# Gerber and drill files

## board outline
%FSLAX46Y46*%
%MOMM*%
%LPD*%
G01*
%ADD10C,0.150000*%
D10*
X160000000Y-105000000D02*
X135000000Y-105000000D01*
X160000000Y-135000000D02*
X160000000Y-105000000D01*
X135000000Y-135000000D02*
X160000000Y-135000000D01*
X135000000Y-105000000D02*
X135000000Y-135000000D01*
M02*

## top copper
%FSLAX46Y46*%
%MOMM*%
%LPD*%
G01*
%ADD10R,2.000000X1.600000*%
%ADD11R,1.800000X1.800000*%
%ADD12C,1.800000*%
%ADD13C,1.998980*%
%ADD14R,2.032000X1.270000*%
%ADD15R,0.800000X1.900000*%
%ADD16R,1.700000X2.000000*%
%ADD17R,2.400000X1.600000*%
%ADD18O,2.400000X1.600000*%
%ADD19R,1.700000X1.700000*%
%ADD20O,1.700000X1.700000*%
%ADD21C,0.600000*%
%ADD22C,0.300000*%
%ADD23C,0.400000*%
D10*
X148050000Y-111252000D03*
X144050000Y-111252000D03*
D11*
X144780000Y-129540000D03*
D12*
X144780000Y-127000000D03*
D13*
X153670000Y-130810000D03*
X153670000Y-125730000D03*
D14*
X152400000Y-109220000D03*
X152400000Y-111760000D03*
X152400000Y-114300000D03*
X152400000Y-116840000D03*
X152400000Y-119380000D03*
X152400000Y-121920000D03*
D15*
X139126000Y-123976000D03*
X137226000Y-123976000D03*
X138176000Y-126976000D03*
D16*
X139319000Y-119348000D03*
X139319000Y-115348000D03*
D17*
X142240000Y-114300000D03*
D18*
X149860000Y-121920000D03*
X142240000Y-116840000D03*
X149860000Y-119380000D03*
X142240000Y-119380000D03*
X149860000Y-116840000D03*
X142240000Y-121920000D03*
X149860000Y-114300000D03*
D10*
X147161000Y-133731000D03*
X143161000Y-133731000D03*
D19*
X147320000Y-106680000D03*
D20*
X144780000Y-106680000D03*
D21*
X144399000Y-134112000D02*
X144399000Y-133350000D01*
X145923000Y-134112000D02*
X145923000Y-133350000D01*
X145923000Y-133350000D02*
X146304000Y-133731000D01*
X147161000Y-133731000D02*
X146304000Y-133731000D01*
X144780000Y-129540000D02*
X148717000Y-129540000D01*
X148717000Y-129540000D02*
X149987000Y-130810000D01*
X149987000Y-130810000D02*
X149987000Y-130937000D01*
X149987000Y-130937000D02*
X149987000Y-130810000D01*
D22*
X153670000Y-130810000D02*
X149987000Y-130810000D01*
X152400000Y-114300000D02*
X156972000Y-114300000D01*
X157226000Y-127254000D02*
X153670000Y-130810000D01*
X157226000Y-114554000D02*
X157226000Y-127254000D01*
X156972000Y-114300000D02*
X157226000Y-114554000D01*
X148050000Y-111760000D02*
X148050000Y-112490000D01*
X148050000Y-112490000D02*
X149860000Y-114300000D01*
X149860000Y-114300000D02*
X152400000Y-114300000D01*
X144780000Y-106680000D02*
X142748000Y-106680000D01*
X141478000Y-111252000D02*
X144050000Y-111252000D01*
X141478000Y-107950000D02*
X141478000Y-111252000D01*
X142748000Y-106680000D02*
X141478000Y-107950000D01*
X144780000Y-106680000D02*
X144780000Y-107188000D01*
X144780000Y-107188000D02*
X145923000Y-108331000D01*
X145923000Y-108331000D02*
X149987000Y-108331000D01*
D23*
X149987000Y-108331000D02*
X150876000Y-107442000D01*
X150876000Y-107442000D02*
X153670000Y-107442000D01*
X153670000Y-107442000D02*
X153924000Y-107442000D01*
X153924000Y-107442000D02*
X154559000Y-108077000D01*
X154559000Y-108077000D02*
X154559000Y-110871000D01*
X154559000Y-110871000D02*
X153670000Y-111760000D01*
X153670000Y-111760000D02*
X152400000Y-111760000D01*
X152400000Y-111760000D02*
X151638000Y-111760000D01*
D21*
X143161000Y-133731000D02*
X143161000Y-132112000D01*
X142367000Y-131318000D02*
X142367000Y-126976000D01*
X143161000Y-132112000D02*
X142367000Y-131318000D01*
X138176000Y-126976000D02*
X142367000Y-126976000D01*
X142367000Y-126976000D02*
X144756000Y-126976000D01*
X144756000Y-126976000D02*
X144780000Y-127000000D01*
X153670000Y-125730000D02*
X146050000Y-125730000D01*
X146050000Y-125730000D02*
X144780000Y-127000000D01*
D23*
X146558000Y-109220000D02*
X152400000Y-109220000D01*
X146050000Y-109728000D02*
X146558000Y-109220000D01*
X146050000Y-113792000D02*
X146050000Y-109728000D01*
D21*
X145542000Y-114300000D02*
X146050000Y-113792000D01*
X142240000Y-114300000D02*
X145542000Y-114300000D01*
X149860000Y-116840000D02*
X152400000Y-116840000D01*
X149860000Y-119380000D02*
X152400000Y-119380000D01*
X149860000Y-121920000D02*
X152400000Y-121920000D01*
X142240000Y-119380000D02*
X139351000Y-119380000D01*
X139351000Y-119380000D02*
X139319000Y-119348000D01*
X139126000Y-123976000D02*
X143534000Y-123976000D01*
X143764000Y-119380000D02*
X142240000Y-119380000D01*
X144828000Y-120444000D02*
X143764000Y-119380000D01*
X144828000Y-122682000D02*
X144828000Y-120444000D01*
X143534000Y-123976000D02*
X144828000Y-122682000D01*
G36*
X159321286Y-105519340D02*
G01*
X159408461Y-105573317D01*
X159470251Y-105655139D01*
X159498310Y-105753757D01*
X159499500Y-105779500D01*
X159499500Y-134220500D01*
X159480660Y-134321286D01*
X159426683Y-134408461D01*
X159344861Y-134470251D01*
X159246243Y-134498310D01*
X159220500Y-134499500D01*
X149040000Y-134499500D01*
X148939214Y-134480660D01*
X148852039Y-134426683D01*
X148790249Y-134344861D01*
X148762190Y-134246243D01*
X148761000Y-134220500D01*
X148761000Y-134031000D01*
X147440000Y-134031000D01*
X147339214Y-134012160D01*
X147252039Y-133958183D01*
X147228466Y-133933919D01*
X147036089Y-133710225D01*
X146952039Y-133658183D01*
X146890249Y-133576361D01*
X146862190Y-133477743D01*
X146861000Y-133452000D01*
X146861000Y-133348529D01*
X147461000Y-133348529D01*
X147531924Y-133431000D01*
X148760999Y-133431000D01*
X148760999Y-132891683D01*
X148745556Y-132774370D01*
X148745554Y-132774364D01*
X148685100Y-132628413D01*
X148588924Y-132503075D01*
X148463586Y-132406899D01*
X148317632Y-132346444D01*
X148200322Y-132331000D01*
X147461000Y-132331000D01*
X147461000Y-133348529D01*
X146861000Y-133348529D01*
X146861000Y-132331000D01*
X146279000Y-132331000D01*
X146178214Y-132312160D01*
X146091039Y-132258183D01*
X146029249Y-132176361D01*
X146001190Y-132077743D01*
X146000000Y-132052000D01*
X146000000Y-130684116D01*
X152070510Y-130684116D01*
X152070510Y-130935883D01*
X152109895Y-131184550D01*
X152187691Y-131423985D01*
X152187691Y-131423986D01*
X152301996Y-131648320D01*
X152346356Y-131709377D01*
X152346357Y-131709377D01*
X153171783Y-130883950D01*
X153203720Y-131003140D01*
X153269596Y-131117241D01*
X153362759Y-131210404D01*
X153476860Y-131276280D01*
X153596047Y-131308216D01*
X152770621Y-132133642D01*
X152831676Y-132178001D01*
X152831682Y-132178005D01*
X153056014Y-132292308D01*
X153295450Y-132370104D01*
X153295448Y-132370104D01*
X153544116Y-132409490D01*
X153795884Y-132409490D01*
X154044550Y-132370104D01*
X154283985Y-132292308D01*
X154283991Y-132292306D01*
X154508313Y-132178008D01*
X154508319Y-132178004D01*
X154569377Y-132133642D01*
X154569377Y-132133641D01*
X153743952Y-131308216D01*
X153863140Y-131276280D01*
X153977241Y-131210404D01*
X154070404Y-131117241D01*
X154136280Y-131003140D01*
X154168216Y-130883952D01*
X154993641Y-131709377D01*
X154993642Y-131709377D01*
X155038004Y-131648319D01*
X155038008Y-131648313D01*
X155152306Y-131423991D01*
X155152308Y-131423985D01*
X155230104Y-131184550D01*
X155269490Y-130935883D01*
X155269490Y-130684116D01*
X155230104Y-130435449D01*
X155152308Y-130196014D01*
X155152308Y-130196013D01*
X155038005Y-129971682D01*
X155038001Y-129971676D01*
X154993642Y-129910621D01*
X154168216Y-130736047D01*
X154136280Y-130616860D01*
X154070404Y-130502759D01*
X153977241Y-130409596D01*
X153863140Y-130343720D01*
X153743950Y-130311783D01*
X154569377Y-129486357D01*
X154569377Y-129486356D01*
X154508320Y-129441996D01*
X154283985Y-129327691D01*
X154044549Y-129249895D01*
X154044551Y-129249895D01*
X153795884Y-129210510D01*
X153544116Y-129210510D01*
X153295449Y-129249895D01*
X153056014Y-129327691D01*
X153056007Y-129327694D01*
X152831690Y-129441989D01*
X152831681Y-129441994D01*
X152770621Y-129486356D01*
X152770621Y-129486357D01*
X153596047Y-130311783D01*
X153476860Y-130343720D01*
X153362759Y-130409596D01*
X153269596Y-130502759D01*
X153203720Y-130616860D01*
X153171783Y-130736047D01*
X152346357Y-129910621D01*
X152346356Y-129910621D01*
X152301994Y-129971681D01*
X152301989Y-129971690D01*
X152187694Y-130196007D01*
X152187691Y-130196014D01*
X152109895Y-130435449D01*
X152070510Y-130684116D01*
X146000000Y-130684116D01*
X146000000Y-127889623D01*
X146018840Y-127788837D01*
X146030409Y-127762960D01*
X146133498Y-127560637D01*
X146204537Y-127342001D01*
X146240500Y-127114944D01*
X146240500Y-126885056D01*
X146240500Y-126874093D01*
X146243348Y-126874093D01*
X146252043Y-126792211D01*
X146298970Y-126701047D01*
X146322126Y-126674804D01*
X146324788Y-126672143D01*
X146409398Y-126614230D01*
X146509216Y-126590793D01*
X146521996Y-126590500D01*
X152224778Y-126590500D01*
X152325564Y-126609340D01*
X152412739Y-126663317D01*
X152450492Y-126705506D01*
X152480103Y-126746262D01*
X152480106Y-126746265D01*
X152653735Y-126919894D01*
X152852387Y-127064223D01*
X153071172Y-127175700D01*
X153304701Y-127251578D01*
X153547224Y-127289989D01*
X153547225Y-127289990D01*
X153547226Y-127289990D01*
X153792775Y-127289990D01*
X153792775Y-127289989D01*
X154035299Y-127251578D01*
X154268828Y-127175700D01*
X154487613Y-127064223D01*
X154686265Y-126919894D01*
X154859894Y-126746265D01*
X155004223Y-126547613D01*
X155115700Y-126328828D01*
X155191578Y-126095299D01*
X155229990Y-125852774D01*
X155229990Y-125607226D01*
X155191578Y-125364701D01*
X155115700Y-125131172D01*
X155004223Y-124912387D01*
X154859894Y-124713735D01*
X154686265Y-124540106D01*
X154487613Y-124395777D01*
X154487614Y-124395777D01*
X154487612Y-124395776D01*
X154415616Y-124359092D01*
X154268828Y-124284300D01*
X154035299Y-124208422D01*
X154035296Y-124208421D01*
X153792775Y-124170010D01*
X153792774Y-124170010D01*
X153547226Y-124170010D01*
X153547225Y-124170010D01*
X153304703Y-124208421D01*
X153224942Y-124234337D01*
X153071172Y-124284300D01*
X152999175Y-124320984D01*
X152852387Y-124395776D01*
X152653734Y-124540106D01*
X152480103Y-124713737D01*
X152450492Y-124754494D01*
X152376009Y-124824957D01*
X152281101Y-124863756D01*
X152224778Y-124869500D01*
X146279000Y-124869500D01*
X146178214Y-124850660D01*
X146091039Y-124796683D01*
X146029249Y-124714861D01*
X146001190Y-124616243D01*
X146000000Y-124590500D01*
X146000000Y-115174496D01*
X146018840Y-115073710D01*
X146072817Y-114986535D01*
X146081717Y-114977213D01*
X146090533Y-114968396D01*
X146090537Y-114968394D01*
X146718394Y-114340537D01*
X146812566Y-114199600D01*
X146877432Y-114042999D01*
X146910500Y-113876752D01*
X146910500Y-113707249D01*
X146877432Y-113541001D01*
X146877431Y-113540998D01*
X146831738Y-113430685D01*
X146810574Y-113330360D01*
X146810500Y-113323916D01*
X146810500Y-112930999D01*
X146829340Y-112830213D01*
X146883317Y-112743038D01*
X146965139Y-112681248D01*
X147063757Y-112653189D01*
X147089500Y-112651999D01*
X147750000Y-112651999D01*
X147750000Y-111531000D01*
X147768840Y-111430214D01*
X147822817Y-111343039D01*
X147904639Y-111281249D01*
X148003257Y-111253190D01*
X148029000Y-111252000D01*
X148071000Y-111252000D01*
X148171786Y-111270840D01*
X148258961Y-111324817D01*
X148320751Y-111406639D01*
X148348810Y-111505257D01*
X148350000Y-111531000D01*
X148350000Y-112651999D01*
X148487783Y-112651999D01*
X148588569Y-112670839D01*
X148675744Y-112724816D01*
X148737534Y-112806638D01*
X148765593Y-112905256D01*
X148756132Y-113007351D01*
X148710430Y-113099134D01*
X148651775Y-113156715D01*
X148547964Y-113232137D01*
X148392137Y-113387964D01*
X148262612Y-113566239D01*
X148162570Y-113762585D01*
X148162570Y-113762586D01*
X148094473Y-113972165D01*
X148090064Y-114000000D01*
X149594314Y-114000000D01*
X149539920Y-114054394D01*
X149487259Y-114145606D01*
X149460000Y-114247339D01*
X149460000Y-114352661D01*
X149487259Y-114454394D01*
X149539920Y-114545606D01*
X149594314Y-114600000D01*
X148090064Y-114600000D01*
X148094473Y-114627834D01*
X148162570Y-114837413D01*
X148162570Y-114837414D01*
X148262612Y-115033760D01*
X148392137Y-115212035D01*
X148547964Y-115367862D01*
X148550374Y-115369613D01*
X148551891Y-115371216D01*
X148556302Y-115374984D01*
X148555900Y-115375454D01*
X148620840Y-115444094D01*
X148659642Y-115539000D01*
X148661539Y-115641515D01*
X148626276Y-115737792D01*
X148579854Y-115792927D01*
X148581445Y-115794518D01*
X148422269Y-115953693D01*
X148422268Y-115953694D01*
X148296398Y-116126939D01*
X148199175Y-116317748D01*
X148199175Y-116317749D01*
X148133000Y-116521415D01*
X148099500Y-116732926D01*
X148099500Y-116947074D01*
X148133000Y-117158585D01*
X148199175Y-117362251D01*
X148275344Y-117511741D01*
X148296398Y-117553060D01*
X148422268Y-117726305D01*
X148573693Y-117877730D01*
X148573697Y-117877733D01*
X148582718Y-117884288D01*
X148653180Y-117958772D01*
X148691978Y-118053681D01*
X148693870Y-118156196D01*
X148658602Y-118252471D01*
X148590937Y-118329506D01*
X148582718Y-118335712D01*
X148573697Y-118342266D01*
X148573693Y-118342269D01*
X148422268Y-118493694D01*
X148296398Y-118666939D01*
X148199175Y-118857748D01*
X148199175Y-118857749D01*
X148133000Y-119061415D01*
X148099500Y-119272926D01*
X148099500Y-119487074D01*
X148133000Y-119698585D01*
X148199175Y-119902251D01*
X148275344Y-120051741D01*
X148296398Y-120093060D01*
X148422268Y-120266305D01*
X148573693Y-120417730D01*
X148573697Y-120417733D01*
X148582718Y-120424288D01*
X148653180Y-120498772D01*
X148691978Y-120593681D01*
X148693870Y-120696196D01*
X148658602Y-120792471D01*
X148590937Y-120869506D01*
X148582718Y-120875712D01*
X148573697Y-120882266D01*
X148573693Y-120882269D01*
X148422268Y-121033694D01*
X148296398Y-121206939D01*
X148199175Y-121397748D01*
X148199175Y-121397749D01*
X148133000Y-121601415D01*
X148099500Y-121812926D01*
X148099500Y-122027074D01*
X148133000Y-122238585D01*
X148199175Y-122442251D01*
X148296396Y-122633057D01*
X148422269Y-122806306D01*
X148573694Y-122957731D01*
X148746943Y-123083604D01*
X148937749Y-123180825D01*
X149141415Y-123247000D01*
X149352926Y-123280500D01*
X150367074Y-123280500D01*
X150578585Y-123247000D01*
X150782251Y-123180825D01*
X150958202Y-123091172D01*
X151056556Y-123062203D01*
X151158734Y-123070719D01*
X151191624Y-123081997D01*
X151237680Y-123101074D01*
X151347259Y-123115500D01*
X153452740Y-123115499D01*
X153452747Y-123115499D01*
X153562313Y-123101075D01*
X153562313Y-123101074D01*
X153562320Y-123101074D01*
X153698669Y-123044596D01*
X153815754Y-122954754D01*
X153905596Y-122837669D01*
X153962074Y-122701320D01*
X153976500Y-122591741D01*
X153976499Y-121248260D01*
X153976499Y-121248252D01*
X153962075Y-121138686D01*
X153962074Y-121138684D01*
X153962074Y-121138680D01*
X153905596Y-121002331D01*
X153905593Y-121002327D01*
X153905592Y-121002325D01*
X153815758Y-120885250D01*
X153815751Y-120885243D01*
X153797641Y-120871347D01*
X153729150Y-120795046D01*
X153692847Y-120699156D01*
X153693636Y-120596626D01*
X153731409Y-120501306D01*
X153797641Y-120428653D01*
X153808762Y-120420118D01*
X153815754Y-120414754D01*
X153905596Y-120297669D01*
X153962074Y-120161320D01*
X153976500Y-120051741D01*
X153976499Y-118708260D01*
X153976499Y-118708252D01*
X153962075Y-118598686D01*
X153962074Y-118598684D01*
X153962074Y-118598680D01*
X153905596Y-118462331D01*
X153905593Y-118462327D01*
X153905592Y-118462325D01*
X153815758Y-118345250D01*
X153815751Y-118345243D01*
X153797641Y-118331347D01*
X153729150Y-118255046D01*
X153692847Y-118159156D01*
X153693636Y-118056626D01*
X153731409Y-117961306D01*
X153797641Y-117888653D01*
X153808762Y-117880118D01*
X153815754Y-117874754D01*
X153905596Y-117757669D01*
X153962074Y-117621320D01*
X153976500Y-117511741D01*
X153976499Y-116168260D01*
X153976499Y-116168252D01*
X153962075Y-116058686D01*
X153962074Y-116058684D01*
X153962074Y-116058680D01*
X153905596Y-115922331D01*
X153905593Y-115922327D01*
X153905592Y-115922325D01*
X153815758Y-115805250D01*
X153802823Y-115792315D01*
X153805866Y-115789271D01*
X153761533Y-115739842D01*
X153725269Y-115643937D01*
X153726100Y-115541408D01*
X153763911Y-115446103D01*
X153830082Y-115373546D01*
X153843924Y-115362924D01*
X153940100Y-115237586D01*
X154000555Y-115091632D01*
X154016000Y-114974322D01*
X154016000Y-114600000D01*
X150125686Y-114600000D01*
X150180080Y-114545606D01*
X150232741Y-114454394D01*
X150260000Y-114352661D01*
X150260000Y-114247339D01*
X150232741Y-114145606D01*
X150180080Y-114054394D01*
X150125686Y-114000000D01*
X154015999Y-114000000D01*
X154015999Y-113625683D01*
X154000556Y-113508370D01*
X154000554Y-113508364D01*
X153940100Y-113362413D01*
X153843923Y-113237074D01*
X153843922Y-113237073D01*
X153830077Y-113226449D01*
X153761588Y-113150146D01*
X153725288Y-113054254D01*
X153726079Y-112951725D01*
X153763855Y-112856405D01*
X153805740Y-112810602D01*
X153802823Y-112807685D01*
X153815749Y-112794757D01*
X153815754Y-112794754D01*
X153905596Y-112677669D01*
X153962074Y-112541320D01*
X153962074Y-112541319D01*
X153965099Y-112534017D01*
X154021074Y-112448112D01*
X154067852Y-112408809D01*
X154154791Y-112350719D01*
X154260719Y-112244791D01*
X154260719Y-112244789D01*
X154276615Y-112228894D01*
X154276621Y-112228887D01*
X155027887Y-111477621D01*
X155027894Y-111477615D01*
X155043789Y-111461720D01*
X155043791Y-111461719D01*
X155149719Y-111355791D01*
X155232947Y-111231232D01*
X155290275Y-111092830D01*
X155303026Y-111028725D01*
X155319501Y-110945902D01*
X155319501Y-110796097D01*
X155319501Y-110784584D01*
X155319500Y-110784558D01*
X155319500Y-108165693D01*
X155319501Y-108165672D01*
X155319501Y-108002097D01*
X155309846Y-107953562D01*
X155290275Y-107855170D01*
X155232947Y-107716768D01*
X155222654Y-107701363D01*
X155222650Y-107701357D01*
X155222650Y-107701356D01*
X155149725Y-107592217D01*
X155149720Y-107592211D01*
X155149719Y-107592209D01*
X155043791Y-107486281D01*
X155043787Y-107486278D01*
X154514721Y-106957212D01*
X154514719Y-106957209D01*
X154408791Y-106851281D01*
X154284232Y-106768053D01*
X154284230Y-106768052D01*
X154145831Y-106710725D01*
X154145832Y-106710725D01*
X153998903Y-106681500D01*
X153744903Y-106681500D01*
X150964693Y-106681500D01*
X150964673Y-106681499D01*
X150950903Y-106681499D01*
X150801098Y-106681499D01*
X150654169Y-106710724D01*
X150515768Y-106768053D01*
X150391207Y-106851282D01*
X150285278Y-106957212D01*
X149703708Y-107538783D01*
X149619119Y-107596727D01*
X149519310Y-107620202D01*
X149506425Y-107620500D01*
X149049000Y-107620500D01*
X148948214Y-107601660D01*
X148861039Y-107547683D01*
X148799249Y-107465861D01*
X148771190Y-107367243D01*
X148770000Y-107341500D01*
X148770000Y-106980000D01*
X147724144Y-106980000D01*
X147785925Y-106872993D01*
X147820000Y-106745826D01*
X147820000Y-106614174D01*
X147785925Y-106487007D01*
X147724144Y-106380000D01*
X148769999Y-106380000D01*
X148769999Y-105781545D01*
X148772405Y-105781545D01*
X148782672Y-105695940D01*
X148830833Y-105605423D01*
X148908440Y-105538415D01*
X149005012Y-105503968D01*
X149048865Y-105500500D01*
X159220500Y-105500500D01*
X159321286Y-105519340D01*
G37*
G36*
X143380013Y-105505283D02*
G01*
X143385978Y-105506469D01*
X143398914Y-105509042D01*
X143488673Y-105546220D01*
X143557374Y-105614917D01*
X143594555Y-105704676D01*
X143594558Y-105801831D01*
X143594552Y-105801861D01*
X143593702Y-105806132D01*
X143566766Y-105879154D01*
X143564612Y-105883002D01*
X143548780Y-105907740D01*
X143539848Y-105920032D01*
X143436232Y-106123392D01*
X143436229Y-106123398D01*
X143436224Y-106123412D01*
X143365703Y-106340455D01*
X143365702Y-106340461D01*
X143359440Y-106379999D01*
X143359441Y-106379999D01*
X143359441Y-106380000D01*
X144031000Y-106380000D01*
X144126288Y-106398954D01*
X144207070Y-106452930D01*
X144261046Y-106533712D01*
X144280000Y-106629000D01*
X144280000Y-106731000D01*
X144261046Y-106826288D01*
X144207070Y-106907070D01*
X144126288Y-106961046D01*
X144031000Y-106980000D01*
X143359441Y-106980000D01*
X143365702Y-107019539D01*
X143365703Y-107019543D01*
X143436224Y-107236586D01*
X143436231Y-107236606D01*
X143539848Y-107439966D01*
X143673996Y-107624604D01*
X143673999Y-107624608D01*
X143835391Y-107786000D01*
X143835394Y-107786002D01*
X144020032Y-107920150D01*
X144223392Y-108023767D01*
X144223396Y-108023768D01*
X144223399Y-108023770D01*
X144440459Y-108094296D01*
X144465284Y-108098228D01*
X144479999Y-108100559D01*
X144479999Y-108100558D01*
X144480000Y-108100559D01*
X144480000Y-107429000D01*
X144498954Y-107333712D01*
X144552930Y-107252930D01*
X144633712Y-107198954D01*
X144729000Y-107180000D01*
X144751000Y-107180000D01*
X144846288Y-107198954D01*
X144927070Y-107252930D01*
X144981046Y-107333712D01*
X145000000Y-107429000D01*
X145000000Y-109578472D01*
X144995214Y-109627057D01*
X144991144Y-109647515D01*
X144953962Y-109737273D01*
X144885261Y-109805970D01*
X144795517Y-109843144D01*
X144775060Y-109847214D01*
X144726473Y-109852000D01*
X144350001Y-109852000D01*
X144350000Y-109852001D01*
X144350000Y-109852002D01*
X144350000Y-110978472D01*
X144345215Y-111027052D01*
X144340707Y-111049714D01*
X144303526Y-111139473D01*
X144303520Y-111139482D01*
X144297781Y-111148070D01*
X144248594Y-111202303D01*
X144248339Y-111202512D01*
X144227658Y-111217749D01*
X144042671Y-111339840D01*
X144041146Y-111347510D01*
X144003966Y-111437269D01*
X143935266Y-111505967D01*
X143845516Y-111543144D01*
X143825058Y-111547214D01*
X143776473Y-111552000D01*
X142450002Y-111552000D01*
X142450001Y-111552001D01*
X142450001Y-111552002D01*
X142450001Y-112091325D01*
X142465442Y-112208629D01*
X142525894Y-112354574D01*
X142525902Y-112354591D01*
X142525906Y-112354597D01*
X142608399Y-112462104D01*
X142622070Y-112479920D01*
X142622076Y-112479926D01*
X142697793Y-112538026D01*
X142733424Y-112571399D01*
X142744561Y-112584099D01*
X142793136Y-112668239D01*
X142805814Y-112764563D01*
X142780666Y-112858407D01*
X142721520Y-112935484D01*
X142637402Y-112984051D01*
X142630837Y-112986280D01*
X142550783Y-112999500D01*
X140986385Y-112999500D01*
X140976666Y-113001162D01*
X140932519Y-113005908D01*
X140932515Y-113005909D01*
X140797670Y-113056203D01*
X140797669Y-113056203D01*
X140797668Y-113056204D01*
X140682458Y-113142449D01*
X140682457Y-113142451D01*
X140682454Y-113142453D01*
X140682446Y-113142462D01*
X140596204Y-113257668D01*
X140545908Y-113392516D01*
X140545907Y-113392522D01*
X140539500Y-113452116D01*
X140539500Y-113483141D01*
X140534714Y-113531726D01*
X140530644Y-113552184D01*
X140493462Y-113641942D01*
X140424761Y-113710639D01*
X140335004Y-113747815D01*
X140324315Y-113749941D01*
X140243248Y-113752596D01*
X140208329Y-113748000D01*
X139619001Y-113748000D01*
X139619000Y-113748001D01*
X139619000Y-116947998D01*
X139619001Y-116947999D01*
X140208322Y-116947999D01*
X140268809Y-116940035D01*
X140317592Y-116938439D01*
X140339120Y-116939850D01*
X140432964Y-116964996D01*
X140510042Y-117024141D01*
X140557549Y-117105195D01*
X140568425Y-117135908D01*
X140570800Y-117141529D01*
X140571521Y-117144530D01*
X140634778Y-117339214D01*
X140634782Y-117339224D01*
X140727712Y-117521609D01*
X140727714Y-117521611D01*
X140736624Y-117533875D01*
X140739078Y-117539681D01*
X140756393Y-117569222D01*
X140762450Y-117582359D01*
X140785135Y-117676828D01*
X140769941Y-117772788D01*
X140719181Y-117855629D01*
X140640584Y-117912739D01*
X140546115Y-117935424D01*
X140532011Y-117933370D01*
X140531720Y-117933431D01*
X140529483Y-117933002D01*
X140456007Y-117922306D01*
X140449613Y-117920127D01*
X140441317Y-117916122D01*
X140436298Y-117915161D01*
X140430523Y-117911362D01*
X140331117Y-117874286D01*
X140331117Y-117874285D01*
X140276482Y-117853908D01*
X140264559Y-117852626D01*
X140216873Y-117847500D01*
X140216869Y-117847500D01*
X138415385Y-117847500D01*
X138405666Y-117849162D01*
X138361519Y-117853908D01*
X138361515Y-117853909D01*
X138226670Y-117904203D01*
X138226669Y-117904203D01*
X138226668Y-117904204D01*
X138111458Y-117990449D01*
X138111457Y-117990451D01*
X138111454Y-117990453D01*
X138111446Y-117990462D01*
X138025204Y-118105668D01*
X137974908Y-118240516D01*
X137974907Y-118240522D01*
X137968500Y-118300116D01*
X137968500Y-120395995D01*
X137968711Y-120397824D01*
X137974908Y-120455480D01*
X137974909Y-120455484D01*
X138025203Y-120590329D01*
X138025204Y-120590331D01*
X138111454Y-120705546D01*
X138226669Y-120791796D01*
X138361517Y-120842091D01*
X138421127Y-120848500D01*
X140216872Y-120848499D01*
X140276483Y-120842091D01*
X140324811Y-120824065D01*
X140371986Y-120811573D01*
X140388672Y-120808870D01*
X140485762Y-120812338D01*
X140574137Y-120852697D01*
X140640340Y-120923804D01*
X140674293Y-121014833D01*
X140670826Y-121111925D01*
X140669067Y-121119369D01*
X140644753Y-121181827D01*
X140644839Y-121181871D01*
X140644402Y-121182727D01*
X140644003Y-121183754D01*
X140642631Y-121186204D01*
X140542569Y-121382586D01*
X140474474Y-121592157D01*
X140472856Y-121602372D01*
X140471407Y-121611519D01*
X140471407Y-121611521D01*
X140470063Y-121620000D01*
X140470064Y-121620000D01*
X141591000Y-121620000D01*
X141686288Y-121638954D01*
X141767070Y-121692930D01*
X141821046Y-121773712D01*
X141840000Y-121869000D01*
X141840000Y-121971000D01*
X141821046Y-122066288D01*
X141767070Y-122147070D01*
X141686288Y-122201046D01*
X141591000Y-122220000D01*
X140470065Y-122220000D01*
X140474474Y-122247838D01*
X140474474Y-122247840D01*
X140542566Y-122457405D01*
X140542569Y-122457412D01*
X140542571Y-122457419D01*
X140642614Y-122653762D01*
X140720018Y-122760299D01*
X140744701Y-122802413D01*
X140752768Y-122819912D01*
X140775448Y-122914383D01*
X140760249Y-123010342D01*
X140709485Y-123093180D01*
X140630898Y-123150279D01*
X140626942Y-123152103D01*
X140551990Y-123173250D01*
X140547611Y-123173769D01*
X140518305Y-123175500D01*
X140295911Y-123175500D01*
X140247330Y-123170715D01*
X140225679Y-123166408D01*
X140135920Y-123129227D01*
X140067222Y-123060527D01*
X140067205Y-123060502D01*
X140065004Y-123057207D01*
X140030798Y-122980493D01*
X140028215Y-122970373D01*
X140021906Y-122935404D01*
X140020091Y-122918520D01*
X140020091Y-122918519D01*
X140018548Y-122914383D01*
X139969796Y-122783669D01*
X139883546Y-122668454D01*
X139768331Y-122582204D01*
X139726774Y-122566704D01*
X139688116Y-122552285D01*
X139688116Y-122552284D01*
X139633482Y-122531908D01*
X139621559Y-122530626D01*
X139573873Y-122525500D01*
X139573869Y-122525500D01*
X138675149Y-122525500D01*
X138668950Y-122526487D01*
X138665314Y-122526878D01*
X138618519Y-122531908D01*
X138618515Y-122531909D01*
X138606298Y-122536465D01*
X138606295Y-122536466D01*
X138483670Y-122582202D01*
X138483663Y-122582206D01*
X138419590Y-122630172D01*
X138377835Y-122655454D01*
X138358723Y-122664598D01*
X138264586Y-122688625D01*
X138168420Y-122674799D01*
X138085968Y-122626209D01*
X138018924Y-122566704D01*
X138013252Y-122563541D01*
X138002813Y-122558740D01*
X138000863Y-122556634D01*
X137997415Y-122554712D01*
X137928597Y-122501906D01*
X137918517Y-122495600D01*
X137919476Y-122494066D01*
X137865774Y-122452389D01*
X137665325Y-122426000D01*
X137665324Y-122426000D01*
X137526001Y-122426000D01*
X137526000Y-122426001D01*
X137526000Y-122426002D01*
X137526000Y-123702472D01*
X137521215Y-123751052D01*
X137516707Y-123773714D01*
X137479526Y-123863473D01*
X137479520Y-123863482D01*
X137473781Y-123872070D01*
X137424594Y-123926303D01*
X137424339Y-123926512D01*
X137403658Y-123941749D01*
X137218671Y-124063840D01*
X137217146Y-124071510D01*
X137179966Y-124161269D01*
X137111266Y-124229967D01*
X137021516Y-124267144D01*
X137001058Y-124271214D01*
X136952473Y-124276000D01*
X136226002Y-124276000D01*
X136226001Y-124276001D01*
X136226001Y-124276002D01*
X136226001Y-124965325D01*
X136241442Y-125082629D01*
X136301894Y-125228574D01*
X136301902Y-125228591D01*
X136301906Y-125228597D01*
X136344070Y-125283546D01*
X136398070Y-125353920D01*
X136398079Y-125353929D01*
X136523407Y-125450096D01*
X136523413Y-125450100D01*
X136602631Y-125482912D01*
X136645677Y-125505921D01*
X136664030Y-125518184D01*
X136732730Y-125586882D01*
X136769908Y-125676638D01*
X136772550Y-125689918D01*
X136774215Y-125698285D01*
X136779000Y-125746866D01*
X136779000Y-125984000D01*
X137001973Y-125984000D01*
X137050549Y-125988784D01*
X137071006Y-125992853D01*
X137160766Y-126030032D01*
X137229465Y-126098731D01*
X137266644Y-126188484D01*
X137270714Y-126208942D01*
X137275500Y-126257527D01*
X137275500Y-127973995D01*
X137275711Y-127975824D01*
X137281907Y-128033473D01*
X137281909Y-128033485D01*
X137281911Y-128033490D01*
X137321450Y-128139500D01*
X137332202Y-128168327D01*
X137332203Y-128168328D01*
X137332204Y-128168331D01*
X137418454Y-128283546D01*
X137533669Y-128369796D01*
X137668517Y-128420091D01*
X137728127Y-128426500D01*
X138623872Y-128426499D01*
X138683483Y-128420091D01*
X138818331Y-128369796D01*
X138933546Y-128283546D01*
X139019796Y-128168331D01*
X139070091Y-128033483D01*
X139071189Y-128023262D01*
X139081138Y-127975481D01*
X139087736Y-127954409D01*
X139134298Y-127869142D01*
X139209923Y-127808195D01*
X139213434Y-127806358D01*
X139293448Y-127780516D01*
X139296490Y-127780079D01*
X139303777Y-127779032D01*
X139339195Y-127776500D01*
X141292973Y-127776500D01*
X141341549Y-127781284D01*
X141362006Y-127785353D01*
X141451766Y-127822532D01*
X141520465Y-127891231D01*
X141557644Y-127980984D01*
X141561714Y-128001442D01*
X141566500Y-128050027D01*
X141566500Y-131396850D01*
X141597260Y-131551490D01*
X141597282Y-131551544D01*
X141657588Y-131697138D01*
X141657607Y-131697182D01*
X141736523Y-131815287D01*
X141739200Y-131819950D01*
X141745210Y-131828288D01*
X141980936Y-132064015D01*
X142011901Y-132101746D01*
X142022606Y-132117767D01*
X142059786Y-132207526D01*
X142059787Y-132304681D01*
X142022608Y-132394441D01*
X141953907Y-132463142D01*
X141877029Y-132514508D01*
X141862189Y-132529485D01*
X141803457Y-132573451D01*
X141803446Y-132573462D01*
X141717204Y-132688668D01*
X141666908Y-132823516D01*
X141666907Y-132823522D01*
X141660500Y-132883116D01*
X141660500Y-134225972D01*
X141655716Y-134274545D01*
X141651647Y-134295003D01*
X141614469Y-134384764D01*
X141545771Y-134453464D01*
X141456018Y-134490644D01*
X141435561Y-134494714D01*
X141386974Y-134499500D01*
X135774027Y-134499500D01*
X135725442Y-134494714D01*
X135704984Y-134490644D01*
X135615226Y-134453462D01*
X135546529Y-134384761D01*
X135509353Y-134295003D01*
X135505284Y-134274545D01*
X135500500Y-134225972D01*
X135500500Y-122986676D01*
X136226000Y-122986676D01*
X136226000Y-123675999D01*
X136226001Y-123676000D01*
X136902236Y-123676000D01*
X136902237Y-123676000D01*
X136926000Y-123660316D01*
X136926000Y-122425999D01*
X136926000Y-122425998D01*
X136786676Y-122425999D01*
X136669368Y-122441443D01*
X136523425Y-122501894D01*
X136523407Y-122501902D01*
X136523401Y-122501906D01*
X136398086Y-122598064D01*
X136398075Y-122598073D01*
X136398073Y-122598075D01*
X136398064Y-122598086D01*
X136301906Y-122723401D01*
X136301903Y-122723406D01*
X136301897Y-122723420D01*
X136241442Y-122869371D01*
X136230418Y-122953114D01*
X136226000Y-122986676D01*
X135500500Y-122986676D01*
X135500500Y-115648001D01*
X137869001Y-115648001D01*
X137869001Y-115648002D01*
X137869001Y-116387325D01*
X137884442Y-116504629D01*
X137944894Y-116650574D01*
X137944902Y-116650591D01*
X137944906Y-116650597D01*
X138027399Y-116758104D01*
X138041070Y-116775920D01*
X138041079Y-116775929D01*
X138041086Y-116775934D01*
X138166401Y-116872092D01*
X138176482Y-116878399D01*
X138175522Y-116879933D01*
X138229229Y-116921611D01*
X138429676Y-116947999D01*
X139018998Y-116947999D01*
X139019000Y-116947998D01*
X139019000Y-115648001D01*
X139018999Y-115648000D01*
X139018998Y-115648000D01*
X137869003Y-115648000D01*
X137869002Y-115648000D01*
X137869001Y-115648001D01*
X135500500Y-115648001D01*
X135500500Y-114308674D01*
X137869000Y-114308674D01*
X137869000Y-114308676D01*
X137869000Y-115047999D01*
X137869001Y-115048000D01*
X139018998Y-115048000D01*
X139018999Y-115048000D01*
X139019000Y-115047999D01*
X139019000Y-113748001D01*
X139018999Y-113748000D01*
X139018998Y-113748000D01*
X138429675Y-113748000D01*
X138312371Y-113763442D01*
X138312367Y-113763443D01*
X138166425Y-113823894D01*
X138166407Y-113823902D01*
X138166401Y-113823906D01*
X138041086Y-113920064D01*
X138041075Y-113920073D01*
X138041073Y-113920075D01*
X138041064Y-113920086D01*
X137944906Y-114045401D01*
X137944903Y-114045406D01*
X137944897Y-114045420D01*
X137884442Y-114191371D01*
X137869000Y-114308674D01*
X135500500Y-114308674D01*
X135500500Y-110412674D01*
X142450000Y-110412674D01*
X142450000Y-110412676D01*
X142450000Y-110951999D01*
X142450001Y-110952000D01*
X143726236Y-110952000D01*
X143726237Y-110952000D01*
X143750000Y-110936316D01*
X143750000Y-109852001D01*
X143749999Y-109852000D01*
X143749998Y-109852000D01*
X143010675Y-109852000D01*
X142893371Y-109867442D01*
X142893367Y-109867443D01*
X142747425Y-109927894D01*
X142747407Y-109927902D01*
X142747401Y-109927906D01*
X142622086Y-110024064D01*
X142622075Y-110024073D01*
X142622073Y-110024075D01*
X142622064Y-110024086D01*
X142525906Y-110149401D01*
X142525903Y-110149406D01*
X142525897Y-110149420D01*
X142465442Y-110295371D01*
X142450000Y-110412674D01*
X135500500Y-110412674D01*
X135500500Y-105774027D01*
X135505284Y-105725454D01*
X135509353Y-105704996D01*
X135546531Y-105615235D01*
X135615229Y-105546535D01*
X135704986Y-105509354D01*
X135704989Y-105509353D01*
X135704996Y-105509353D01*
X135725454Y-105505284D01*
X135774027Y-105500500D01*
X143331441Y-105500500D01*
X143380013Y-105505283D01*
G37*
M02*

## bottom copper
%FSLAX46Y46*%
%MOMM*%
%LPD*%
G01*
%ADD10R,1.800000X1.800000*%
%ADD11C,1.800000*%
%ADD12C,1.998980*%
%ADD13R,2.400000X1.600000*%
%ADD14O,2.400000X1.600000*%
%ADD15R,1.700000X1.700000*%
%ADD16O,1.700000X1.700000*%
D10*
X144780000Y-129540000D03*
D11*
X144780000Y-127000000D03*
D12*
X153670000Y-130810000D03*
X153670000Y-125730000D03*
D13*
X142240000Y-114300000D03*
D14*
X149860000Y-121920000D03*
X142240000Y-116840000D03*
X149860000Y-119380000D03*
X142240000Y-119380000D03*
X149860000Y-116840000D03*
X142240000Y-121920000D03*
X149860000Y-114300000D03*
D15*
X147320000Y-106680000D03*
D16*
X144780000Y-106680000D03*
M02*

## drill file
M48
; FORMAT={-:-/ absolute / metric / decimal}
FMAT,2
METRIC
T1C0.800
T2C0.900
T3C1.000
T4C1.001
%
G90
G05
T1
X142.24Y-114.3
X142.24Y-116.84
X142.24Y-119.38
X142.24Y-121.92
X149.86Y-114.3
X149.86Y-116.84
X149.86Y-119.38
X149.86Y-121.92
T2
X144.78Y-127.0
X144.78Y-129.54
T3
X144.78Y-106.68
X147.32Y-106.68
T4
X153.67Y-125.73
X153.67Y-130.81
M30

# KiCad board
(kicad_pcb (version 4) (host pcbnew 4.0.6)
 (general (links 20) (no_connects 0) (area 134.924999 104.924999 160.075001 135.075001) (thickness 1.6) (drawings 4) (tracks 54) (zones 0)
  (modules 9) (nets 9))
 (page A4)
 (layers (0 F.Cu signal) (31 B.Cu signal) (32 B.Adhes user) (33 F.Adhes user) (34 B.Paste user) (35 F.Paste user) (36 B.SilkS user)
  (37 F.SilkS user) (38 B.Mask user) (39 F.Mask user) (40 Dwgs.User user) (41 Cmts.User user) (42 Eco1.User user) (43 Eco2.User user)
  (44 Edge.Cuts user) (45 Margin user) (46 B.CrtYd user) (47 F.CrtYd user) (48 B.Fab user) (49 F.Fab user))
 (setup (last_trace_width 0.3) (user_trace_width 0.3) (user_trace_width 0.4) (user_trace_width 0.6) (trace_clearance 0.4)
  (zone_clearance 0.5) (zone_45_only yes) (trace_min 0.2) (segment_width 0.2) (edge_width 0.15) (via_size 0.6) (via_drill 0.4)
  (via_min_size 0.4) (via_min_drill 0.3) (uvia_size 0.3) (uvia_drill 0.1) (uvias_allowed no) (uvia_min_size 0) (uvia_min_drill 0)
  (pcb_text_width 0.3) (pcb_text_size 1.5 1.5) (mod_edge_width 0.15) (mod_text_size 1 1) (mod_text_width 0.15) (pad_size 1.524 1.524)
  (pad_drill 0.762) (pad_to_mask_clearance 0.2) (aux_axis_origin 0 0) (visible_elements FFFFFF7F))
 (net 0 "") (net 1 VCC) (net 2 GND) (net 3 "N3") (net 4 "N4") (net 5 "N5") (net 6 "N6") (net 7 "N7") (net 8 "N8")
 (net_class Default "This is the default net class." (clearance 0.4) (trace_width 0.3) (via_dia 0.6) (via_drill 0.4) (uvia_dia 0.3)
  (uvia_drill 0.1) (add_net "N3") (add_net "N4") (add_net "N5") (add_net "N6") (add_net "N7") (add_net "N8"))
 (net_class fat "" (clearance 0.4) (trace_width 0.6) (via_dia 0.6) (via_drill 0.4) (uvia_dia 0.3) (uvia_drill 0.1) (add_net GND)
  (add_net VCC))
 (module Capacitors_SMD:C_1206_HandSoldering (layer F.Cu) (at 146.05 111.252 180)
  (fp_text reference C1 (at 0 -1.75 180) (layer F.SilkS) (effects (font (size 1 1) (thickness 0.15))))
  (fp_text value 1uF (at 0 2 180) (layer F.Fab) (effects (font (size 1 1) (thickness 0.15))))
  (pad 1 smd rect (at -2 0 180) (size 2 1.6) (layers F.Cu F.Paste F.Mask) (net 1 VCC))
  (pad 2 smd rect (at 2 0 180) (size 2 1.6) (layers F.Cu F.Paste F.Mask) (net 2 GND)))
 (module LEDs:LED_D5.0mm (layer F.Cu) (at 144.78 129.54 90)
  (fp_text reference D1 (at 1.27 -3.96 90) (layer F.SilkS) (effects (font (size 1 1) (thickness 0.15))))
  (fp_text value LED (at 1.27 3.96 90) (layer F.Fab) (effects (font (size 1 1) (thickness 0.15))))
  (pad 1 thru_hole rect (at 0 0 90) (size 1.8 1.8) (drill 0.9) (layers *.Cu *.Mask) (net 1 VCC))
  (pad 2 thru_hole circle (at 2.54 0 90) (size 1.8 1.8) (drill 0.9) (layers *.Cu *.Mask) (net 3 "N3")))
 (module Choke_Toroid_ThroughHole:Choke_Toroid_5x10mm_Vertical (layer F.Cu) (at 148.59 130.81)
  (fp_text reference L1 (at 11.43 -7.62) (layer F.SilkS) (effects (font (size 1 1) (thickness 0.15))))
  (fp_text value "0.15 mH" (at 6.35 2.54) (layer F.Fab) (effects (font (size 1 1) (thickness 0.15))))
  (pad 1 thru_hole circle (at 5.08 0) (size 1.99898 1.99898) (drill 1.00076) (layers *.Cu *.Mask) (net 1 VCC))
  (pad 2 thru_hole circle (at 5.08 -5.08) (size 1.99898 1.99898) (drill 1.00076) (layers *.Cu *.Mask) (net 3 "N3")))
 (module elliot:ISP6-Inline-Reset (layer F.Cu) (at 152.4 116.84 270)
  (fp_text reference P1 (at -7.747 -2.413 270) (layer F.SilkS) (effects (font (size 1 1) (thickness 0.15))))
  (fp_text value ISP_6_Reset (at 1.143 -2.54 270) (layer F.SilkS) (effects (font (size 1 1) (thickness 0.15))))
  (pad 1 smd rect (at -7.62 0 270) (size 1.27 2.032) (layers F.Cu F.Paste F.Mask) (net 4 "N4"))
  (pad 2 smd rect (at -5.08 0 270) (size 1.27 2.032) (layers F.Cu F.Paste F.Mask) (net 2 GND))
  (pad 3 smd rect (at -2.54 0 270) (size 1.27 2.032) (layers F.Cu F.Paste F.Mask) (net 1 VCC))
  (pad 4 smd rect (at 0 0 270) (size 1.27 2.032) (layers F.Cu F.Paste F.Mask) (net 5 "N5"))
  (pad 5 smd rect (at 2.54 0 270) (size 1.27 2.032) (layers F.Cu F.Paste F.Mask) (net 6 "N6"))
  (pad 6 smd rect (at 5.08 0 270) (size 1.27 2.032) (layers F.Cu F.Paste F.Mask) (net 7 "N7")))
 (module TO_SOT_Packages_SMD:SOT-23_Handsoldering (layer F.Cu) (at 138.176 125.476 270)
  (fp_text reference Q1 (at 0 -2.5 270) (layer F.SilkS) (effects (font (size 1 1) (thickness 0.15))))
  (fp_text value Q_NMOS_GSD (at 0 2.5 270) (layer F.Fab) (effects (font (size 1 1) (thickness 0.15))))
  (pad 1 smd rect (at -1.5 -0.95 270) (size 1.9 0.8) (layers F.Cu F.Paste F.Mask) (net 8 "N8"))
  (pad 2 smd rect (at -1.5 0.95 270) (size 1.9 0.8) (layers F.Cu F.Paste F.Mask) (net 2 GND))
  (pad 3 smd rect (at 1.5 0 270) (size 1.9 0.8) (layers F.Cu F.Paste F.Mask) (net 3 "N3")))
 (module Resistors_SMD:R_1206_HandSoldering (layer F.Cu) (at 139.319 117.348 90)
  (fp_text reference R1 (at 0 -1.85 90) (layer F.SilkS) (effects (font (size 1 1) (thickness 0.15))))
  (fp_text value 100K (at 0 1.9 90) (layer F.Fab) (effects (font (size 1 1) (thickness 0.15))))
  (pad 1 smd rect (at -2 0 90) (size 2 1.7) (layers F.Cu F.Paste F.Mask) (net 8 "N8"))
  (pad 2 smd rect (at 2 0 90) (size 2 1.7) (layers F.Cu F.Paste F.Mask) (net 2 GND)))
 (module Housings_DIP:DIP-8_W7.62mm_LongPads (layer F.Cu) (at 142.24 114.3)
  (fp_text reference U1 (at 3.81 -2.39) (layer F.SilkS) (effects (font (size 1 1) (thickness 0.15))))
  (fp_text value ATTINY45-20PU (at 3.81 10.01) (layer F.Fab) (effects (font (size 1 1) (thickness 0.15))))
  (pad 1 thru_hole rect (at 0 0) (size 2.4 1.6) (drill 0.8) (layers *.Cu *.Mask) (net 4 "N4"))
  (pad 5 thru_hole oval (at 7.62 7.62) (size 2.4 1.6) (drill 0.8) (layers *.Cu *.Mask) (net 7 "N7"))
  (pad 2 thru_hole oval (at 0 2.54) (size 2.4 1.6) (drill 0.8) (layers *.Cu *.Mask))
  (pad 6 thru_hole oval (at 7.62 5.08) (size 2.4 1.6) (drill 0.8) (layers *.Cu *.Mask) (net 6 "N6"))
  (pad 3 thru_hole oval (at 0 5.08) (size 2.4 1.6) (drill 0.8) (layers *.Cu *.Mask) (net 8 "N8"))
  (pad 7 thru_hole oval (at 7.62 2.54) (size 2.4 1.6) (drill 0.8) (layers *.Cu *.Mask) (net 5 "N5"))
  (pad 4 thru_hole oval (at 0 7.62) (size 2.4 1.6) (drill 0.8) (layers *.Cu *.Mask) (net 2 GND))
  (pad 8 thru_hole oval (at 7.62 0) (size 2.4 1.6) (drill 0.8) (layers *.Cu *.Mask) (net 1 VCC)))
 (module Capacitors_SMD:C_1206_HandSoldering (layer F.Cu) (at 145.161 133.731 180)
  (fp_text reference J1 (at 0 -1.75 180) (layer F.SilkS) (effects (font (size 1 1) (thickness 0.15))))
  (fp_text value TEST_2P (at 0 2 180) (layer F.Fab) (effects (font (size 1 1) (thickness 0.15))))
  (pad 1 smd rect (at -2 0 180) (size 2 1.6) (layers F.Cu F.Paste F.Mask) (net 1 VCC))
  (pad 2 smd rect (at 2 0 180) (size 2 1.6) (layers F.Cu F.Paste F.Mask) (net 3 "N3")))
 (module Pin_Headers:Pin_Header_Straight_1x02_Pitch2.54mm (layer F.Cu) (at 147.32 106.68 270)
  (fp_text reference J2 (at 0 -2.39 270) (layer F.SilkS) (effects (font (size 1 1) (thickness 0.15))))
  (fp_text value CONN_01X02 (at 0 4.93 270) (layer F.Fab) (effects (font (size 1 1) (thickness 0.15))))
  (pad 1 thru_hole rect (at 0 0 270) (size 1.7 1.7) (drill 1) (layers *.Cu *.Mask) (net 1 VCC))
  (pad 2 thru_hole oval (at 0 2.54 270) (size 1.7 1.7) (drill 1) (layers *.Cu *.Mask) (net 2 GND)))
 (gr_line (start 160 105) (end 135 105) (angle 90) (layer Edge.Cuts) (width 0.15))
 (gr_line (start 160 135) (end 160 105) (angle 90) (layer Edge.Cuts) (width 0.15))
 (gr_line (start 135 135) (end 160 135) (angle 90) (layer Edge.Cuts) (width 0.15))
 (gr_line (start 135 105) (end 135 135) (angle 90) (layer Edge.Cuts) (width 0.15))
 (segment (start 144.399 134.112) (end 144.399 133.35) (width 0.6) (layer F.Cu) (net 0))
 (segment (start 145.923 134.112) (end 145.923 133.35) (width 0.6) (layer F.Cu) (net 1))
 (segment (start 145.923 133.35) (end 146.304 133.731) (width 0.6) (layer F.Cu) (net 1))
 (segment (start 147.161 133.731) (end 146.304 133.731) (width 0.6) (layer F.Cu) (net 1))
 (segment (start 144.78 129.54) (end 148.717 129.54) (width 0.6) (layer F.Cu) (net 1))
 (segment (start 148.717 129.54) (end 149.987 130.81) (width 0.6) (layer F.Cu) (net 1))
 (segment (start 149.987 130.81) (end 149.987 130.937) (width 0.6) (layer F.Cu) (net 1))
 (segment (start 149.987 130.937) (end 149.987 130.81) (width 0.6) (layer F.Cu) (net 1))
 (segment (start 153.67 130.81) (end 149.987 130.81) (width 0.3) (layer F.Cu) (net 1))
 (segment (start 152.4 114.3) (end 156.972 114.3) (width 0.3) (layer F.Cu) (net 1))
 (segment (start 157.226 127.254) (end 153.67 130.81) (width 0.3) (layer F.Cu) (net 1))
 (segment (start 157.226 114.554) (end 157.226 127.254) (width 0.3) (layer F.Cu) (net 1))
 (segment (start 156.972 114.3) (end 157.226 114.554) (width 0.3) (layer F.Cu) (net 1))
 (segment (start 148.05 111.76) (end 148.05 112.49) (width 0.3) (layer F.Cu) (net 1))
 (segment (start 148.05 112.49) (end 149.86 114.3) (width 0.3) (layer F.Cu) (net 1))
 (segment (start 149.86 114.3) (end 152.4 114.3) (width 0.3) (layer F.Cu) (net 1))
 (segment (start 144.78 106.68) (end 142.748 106.68) (width 0.3) (layer F.Cu) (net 2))
 (segment (start 141.478 111.252) (end 144.05 111.252) (width 0.3) (layer F.Cu) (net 2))
 (segment (start 141.478 107.95) (end 141.478 111.252) (width 0.3) (layer F.Cu) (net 2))
 (segment (start 142.748 106.68) (end 141.478 107.95) (width 0.3) (layer F.Cu) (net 2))
 (segment (start 144.78 106.68) (end 144.78 107.188) (width 0.3) (layer F.Cu) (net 2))
 (segment (start 144.78 107.188) (end 145.923 108.331) (width 0.3) (layer F.Cu) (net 2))
 (segment (start 145.923 108.331) (end 149.987 108.331) (width 0.3) (layer F.Cu) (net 2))
 (segment (start 149.987 108.331) (end 150.876 107.442) (width 0.4) (layer F.Cu) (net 2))
 (segment (start 150.876 107.442) (end 153.67 107.442) (width 0.4) (layer F.Cu) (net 2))
 (segment (start 153.67 107.442) (end 153.924 107.442) (width 0.4) (layer F.Cu) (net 2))
 (segment (start 153.924 107.442) (end 154.559 108.077) (width 0.4) (layer F.Cu) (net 2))
 (segment (start 154.559 108.077) (end 154.559 110.871) (width 0.4) (layer F.Cu) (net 2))
 (segment (start 154.559 110.871) (end 153.67 111.76) (width 0.4) (layer F.Cu) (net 2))
 (segment (start 153.67 111.76) (end 152.4 111.76) (width 0.4) (layer F.Cu) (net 2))
 (segment (start 152.4 111.76) (end 151.638 111.76) (width 0.4) (layer F.Cu) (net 2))
 (segment (start 143.161 133.731) (end 143.161 132.112) (width 0.6) (layer F.Cu) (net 3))
 (segment (start 142.367 131.318) (end 142.367 126.976) (width 0.6) (layer F.Cu) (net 3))
 (segment (start 143.161 132.112) (end 142.367 131.318) (width 0.6) (layer F.Cu) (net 3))
 (segment (start 138.176 126.976) (end 142.367 126.976) (width 0.6) (layer F.Cu) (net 3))
 (segment (start 142.367 126.976) (end 144.756 126.976) (width 0.6) (layer F.Cu) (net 3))
 (segment (start 144.756 126.976) (end 144.78 127) (width 0.6) (layer F.Cu) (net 3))
 (segment (start 153.67 125.73) (end 146.05 125.73) (width 0.6) (layer F.Cu) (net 3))
 (segment (start 146.05 125.73) (end 144.78 127) (width 0.6) (layer F.Cu) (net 3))
 (segment (start 146.558 109.22) (end 152.4 109.22) (width 0.4) (layer F.Cu) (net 4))
 (segment (start 146.05 109.728) (end 146.558 109.22) (width 0.4) (layer F.Cu) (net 4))
 (segment (start 146.05 113.792) (end 146.05 109.728) (width 0.4) (layer F.Cu) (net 4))
 (segment (start 145.542 114.3) (end 146.05 113.792) (width 0.6) (layer F.Cu) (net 4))
 (segment (start 142.24 114.3) (end 145.542 114.3) (width 0.6) (layer F.Cu) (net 4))
 (segment (start 149.86 116.84) (end 152.4 116.84) (width 0.6) (layer F.Cu) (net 5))
 (segment (start 149.86 119.38) (end 152.4 119.38) (width 0.6) (layer F.Cu) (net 6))
 (segment (start 149.86 121.92) (end 152.4 121.92) (width 0.6) (layer F.Cu) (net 7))
 (segment (start 142.24 119.38) (end 139.351 119.38) (width 0.6) (layer F.Cu) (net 8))
 (segment (start 139.351 119.38) (end 139.319 119.348) (width 0.6) (layer F.Cu) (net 8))
 (segment (start 139.126 123.976) (end 143.534 123.976) (width 0.6) (layer F.Cu) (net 8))
 (segment (start 143.764 119.38) (end 142.24 119.38) (width 0.6) (layer F.Cu) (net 8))
 (segment (start 144.828 120.444) (end 143.764 119.38) (width 0.6) (layer F.Cu) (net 8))
 (segment (start 144.828 122.682) (end 144.828 120.444) (width 0.6) (layer F.Cu) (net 8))
 (segment (start 143.534 123.976) (end 144.828 122.682) (width 0.6) (layer F.Cu) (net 8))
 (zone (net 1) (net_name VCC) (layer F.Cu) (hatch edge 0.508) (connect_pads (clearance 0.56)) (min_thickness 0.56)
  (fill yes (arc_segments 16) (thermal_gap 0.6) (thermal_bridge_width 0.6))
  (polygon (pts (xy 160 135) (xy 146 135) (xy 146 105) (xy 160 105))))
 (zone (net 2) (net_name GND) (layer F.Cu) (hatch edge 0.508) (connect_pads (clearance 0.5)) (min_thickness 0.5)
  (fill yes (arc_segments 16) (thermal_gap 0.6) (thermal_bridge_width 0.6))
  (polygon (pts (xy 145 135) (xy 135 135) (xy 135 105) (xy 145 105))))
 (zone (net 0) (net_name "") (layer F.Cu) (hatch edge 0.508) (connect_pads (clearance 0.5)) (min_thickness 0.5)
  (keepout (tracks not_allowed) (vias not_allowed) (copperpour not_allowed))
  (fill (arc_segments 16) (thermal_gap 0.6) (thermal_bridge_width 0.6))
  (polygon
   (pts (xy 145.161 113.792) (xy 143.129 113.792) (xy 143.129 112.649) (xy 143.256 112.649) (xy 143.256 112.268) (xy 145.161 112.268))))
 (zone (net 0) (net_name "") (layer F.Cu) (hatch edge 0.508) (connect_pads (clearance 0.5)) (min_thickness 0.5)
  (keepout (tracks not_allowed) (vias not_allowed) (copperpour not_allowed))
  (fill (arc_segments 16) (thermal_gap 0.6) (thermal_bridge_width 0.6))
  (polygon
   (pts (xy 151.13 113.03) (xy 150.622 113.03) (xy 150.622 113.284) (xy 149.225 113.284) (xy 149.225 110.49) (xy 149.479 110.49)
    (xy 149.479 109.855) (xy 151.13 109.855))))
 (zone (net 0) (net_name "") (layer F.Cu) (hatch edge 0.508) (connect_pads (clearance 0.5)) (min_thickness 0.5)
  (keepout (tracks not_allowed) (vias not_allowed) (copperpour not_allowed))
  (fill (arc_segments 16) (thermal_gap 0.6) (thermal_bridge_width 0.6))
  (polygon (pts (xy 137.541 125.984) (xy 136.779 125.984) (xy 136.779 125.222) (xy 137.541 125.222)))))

